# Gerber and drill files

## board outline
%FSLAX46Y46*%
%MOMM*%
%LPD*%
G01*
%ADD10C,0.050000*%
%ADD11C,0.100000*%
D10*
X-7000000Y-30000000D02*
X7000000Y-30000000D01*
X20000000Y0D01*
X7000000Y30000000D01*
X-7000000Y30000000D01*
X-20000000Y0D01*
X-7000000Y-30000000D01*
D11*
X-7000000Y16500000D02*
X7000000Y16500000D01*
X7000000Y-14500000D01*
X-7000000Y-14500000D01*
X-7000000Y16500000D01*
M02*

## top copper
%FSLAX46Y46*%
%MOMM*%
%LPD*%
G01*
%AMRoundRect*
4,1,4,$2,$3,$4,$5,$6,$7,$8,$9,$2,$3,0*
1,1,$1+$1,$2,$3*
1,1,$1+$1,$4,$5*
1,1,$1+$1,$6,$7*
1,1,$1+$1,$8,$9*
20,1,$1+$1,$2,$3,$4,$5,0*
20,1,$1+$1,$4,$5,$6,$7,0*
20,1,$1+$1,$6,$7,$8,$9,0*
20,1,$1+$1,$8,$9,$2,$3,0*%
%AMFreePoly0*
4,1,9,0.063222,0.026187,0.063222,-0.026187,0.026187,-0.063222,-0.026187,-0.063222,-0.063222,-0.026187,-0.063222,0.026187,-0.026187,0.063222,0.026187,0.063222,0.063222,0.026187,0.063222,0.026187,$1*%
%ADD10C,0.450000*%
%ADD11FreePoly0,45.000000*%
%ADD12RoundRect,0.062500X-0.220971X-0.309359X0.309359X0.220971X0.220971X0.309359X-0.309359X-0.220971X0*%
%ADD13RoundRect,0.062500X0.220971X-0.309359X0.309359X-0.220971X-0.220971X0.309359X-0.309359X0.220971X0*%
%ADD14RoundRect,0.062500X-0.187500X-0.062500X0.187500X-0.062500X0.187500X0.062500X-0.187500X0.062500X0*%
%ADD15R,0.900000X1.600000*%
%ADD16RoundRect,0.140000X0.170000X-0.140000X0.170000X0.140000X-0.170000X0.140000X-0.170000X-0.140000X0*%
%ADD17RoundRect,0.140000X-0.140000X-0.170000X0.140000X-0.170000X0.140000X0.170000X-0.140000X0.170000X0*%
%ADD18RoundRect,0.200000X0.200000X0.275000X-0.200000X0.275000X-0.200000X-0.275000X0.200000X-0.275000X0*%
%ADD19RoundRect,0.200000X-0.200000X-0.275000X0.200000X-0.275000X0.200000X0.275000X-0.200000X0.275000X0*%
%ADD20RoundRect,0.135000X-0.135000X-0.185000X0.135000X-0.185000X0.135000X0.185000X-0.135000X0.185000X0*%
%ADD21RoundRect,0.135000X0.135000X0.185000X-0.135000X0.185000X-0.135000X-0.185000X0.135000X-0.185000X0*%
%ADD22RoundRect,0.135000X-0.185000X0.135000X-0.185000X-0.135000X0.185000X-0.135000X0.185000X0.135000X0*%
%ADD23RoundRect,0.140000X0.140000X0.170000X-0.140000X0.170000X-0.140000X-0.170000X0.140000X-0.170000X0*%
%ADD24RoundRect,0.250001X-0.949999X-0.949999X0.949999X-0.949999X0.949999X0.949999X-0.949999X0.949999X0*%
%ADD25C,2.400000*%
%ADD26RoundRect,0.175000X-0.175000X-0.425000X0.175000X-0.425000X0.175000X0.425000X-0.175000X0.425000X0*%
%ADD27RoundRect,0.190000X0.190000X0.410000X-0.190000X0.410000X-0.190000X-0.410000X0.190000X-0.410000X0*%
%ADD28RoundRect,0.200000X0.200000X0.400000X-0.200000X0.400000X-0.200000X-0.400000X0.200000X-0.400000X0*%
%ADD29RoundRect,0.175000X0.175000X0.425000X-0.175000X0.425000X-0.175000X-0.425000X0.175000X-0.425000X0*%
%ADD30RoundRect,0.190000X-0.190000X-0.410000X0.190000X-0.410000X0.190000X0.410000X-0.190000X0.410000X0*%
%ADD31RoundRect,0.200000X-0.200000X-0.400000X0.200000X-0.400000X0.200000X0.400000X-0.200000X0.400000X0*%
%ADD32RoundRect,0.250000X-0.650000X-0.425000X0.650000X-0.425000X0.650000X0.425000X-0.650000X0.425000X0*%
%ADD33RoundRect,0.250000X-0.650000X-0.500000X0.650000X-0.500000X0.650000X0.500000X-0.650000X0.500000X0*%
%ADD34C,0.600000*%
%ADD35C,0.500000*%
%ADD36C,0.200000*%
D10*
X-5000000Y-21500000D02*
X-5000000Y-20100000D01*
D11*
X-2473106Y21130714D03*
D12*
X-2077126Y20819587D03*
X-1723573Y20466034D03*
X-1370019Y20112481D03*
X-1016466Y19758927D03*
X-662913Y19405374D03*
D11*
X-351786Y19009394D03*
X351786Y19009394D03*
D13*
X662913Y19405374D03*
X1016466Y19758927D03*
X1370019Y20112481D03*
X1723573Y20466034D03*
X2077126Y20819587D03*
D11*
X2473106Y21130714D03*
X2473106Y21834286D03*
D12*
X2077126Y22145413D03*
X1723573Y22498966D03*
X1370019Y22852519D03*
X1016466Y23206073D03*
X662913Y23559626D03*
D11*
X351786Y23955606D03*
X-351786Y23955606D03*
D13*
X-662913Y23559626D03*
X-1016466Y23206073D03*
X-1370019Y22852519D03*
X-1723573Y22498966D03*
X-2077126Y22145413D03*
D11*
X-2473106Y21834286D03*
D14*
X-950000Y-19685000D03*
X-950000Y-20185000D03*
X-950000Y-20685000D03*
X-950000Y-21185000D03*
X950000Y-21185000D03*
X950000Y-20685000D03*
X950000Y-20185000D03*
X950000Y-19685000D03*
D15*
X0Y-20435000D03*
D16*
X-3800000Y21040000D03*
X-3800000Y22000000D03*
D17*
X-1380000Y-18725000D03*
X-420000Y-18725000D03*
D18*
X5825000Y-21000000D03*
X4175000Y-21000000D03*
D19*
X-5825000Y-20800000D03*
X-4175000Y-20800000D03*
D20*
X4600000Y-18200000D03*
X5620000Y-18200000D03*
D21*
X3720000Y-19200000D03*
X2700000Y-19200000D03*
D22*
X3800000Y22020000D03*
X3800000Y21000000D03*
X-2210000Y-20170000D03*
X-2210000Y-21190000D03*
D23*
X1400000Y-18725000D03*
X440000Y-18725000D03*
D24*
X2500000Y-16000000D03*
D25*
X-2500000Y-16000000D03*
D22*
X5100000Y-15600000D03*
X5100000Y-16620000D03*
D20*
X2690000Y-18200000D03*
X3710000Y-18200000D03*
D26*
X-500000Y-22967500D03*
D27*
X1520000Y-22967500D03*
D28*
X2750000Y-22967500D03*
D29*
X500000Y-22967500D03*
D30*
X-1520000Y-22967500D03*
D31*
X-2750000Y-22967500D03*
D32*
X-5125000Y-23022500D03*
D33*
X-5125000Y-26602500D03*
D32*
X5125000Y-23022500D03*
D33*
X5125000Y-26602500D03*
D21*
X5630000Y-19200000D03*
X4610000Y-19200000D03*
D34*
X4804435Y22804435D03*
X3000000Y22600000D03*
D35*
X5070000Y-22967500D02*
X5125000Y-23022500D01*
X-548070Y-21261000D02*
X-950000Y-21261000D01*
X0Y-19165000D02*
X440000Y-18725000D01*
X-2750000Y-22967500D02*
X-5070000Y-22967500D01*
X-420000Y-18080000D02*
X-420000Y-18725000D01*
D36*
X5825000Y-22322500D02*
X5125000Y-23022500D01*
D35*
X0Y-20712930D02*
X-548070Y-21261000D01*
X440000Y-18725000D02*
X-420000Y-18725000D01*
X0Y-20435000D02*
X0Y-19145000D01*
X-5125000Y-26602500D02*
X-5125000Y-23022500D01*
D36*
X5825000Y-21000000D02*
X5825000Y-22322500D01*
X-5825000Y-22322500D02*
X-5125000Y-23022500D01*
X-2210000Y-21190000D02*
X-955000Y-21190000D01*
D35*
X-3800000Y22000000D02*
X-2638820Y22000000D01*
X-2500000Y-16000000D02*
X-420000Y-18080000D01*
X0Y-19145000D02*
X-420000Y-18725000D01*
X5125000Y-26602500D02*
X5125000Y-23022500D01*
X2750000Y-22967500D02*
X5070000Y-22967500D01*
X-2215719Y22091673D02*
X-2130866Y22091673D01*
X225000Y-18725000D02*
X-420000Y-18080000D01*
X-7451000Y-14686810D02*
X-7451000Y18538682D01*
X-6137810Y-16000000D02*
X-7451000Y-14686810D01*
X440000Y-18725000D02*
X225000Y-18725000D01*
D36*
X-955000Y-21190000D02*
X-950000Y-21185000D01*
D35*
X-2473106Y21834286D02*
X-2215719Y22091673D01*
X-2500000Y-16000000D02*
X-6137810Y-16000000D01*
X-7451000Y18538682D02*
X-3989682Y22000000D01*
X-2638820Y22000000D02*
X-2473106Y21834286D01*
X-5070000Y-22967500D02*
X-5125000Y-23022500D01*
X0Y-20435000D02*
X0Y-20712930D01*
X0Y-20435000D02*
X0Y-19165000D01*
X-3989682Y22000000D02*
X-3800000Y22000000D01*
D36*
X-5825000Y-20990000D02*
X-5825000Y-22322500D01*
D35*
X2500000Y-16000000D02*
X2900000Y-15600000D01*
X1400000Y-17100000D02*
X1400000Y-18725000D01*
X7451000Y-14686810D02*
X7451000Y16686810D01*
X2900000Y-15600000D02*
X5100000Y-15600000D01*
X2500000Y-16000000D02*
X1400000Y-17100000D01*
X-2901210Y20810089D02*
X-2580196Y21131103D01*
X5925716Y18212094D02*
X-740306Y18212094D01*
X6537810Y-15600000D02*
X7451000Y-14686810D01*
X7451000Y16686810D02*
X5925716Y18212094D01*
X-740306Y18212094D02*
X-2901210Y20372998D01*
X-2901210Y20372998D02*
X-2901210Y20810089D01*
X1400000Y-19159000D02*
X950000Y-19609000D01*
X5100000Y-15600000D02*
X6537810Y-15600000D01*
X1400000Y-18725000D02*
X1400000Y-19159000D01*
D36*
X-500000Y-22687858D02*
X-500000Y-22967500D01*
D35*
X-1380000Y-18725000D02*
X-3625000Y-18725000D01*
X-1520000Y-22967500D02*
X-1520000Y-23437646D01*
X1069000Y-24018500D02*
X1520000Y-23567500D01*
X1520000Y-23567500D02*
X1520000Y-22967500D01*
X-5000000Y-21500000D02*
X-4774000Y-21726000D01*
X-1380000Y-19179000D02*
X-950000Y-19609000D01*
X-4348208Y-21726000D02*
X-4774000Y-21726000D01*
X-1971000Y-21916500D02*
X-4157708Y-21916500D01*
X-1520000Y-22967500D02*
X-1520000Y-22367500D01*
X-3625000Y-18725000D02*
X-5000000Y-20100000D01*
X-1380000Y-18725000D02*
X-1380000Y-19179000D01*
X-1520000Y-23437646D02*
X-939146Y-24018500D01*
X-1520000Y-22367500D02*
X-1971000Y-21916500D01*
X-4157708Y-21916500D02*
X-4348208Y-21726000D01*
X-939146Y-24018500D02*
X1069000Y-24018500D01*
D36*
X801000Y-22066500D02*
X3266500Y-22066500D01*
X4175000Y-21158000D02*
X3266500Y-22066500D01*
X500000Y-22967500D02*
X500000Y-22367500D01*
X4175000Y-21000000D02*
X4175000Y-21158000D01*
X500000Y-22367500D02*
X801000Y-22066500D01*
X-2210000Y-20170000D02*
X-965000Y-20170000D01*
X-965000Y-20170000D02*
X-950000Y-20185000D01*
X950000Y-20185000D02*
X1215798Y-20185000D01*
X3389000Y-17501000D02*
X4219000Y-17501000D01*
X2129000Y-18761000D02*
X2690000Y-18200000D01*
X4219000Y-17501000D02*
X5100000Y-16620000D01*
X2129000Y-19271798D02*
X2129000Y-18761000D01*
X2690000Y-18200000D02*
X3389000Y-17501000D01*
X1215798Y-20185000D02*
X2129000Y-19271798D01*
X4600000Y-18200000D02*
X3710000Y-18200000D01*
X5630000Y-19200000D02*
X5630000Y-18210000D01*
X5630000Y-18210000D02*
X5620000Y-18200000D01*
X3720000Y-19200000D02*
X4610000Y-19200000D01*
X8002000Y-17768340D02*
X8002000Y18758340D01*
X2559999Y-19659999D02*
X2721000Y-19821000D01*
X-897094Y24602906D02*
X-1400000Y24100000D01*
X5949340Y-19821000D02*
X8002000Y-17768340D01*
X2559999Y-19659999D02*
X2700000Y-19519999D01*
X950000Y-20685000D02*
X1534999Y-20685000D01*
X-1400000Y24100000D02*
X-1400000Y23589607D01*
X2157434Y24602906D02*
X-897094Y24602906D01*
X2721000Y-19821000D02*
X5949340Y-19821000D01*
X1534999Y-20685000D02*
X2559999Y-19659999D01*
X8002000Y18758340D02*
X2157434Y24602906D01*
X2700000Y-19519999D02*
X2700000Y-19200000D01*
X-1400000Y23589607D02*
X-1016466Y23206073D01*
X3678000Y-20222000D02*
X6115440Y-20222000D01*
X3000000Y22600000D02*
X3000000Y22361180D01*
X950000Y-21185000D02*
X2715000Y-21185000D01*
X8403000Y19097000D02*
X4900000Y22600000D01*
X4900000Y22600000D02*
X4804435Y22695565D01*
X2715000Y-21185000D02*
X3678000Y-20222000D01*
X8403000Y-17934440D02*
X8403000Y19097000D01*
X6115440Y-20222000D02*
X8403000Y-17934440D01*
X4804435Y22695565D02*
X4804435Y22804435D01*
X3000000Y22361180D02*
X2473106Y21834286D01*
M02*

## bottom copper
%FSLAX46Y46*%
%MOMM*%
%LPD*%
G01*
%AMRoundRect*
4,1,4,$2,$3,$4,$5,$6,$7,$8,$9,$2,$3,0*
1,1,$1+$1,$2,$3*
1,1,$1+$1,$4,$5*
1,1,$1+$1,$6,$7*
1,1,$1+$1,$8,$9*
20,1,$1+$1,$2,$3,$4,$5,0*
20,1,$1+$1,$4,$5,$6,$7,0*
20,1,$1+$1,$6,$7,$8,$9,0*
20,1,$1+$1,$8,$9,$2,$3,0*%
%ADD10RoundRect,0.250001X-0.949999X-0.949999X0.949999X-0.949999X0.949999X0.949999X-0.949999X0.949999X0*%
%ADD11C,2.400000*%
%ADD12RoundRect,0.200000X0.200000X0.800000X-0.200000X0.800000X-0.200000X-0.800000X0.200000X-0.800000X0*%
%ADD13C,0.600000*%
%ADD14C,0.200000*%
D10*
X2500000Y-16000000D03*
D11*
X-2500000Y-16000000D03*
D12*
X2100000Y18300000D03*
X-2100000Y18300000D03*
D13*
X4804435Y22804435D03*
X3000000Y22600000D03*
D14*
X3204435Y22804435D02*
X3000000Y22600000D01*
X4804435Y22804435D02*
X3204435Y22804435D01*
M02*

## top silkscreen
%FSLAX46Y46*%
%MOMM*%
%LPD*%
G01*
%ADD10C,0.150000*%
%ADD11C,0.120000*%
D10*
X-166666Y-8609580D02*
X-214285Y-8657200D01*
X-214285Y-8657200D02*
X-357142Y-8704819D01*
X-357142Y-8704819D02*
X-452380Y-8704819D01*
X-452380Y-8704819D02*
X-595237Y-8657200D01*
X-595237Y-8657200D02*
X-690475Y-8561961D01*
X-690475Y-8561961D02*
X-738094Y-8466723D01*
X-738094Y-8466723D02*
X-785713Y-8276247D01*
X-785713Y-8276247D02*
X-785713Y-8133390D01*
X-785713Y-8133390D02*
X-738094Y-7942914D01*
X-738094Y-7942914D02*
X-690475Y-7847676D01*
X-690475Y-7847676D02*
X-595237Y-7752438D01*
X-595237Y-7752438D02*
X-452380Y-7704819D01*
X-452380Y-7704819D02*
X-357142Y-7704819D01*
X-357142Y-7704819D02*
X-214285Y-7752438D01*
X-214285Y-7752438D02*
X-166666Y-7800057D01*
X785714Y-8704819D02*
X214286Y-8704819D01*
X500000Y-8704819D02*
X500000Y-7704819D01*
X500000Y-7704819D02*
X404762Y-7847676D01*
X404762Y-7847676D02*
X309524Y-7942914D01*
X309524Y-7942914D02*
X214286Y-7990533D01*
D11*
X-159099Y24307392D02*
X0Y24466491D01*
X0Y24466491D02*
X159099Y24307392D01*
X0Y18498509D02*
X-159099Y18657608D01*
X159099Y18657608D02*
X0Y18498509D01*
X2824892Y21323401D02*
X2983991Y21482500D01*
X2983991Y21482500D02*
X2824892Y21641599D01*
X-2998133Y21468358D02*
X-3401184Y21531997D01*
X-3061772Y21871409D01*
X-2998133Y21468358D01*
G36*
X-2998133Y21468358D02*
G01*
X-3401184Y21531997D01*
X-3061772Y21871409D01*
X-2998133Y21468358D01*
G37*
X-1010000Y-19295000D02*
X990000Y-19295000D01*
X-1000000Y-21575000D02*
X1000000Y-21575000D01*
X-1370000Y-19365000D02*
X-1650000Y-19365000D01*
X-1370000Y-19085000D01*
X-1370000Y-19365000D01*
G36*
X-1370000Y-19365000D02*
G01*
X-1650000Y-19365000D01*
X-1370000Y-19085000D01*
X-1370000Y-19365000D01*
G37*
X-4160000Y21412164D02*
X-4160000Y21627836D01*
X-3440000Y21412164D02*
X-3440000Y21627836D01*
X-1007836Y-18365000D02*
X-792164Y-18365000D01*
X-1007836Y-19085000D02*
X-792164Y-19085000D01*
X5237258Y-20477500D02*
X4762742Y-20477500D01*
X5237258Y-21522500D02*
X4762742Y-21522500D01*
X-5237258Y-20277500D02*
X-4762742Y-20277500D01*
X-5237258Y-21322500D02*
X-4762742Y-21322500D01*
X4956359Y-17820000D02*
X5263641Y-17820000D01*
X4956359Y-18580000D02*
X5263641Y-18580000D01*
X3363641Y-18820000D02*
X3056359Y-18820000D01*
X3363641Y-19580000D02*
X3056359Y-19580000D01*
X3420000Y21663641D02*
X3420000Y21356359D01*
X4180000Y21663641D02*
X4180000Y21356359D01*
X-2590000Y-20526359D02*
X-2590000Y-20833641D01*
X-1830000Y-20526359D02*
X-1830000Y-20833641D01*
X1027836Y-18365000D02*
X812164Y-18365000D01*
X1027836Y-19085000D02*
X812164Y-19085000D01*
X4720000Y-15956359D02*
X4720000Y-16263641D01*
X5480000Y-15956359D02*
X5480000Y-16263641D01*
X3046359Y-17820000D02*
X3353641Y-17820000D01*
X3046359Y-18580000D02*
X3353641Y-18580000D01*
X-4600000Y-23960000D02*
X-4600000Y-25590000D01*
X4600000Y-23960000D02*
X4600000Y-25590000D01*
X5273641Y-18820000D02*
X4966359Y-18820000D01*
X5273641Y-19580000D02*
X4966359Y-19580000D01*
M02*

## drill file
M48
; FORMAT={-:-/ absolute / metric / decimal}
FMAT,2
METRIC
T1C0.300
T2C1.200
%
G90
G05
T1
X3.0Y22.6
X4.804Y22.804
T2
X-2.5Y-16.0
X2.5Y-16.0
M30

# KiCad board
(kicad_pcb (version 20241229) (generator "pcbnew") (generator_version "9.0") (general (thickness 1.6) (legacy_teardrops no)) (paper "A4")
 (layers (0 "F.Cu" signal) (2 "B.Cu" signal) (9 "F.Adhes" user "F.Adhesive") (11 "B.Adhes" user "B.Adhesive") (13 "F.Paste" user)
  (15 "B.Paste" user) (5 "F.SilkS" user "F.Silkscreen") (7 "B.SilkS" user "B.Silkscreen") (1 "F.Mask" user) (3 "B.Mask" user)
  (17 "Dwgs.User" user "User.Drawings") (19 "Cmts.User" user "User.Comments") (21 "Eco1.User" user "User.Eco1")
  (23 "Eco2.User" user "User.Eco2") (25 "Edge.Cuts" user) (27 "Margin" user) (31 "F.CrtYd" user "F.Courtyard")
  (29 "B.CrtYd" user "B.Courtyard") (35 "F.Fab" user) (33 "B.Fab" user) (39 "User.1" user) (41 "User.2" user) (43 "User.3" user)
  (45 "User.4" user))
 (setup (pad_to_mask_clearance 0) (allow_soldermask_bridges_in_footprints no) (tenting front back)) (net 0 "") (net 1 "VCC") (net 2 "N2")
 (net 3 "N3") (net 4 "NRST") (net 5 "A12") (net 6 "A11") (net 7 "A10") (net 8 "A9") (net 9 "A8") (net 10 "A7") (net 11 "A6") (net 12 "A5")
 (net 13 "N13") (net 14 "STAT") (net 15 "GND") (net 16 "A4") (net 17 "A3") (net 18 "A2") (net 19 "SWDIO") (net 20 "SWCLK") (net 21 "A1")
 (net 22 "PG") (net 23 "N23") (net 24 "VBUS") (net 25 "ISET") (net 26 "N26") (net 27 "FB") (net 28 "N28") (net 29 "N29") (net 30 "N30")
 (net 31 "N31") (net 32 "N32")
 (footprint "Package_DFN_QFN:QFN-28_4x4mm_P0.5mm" (layer "F.Cu") (at 0 -21.4825 45)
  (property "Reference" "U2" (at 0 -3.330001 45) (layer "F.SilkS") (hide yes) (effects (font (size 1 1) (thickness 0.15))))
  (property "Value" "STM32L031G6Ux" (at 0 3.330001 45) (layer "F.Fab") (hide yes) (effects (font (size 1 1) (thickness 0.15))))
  (fp_line (start 1.885 -2.11) (end 2.11 -2.11) (stroke (width 0.12) (type solid)) (layer "F.SilkS"))
  (fp_line (start 2.11 -2.11) (end 2.11 -1.885) (stroke (width 0.12) (type solid)) (layer "F.SilkS"))
  (fp_line (start -2.11 2.11) (end -2.11 1.885) (stroke (width 0.12) (type solid)) (layer "F.SilkS"))
  (fp_line (start -1.885 2.11) (end -2.11 2.11) (stroke (width 0.12) (type solid)) (layer "F.SilkS"))
  (fp_line (start 1.885 2.11) (end 2.11 2.11) (stroke (width 0.12) (type solid)) (layer "F.SilkS"))
  (fp_line (start 2.11 2.11) (end 2.11 1.885) (stroke (width 0.12) (type solid)) (layer "F.SilkS"))
  (fp_poly (pts (xy -2.13 -2.11) (xy -2.370001 -2.44) (xy -1.89 -2.44)) (stroke (width 0.12) (type solid)) (fill yes) (layer "F.SilkS"))
  (pad "1" smd custom (at -1.9975 -1.5 45) (size 0.136863 0.136863) (layers "F.Cu" "F.Mask" "F.Paste") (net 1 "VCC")
   (options (clearance outline) (anchor circle)) (primitives))
  (pad "2" smd roundrect (at -1.9375 -1 45) (size 0.875 0.25) (layers "F.Cu" "F.Mask" "F.Paste") (roundrect_rratio 0.25) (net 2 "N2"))
  (pad "3" smd roundrect (at -1.9375 -0.5 45) (size 0.875 0.25) (layers "F.Cu" "F.Mask" "F.Paste") (roundrect_rratio 0.25) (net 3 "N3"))
  (pad "4" smd roundrect (at -1.937499 0 45) (size 0.875 0.25) (layers "F.Cu" "F.Mask" "F.Paste") (roundrect_rratio 0.25) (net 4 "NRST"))
  (pad "5" smd roundrect (at -1.9375 0.5 45) (size 0.875 0.25) (layers "F.Cu" "F.Mask" "F.Paste") (roundrect_rratio 0.25) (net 1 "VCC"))
  (pad "6" smd roundrect (at -1.9375 1 45) (size 0.875 0.25) (layers "F.Cu" "F.Mask" "F.Paste") (roundrect_rratio 0.25) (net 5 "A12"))
  (pad "7" smd custom (at -1.9975 1.5 45) (size 0.136863 0.136863) (layers "F.Cu" "F.Mask" "F.Paste") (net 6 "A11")
   (options (clearance outline) (anchor circle)) (primitives))
  (pad "8" smd custom (at -1.5 1.9975 45) (size 0.136863 0.136863) (layers "F.Cu" "F.Mask" "F.Paste") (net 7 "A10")
   (options (clearance outline) (anchor circle)) (primitives))
  (pad "9" smd roundrect (at -1 1.9375 45) (size 0.25 0.875) (layers "F.Cu" "F.Mask" "F.Paste") (roundrect_rratio 0.25) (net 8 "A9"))
  (pad "10" smd roundrect (at -0.5 1.9375 45) (size 0.25 0.875) (layers "F.Cu" "F.Mask" "F.Paste") (roundrect_rratio 0.25) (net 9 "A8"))
  (pad "11" smd roundrect (at 0 1.937499 45) (size 0.25 0.875) (layers "F.Cu" "F.Mask" "F.Paste") (roundrect_rratio 0.25) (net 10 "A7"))
  (pad "12" smd roundrect (at 0.5 1.9375 45) (size 0.25 0.875) (layers "F.Cu" "F.Mask" "F.Paste") (roundrect_rratio 0.25) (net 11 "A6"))
  (pad "13" smd roundrect (at 1 1.9375 45) (size 0.25 0.875) (layers "F.Cu" "F.Mask" "F.Paste") (roundrect_rratio 0.25) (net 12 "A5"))
  (pad "14" smd custom (at 1.5 1.9975 45) (size 0.136863 0.136863) (layers "F.Cu" "F.Mask" "F.Paste") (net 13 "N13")
   (options (clearance outline) (anchor circle)) (primitives))
  (pad "15" smd custom (at 1.9975 1.5 45) (size 0.136863 0.136863) (layers "F.Cu" "F.Mask" "F.Paste") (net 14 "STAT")
   (options (clearance outline) (anchor circle)) (primitives))
  (pad "16" smd roundrect (at 1.9375 1 45) (size 0.875 0.25) (layers "F.Cu" "F.Mask" "F.Paste") (roundrect_rratio 0.25) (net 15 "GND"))
  (pad "17" smd roundrect (at 1.9375 0.5 45) (size 0.875 0.25) (layers "F.Cu" "F.Mask" "F.Paste") (roundrect_rratio 0.25) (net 1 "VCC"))
  (pad "18" smd roundrect (at 1.937499 0 45) (size 0.875 0.25) (layers "F.Cu" "F.Mask" "F.Paste") (roundrect_rratio 0.25) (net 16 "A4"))
  (pad "19" smd roundrect (at 1.9375 -0.5 45) (size 0.875 0.25) (layers "F.Cu" "F.Mask" "F.Paste") (roundrect_rratio 0.25) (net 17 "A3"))
  (pad "20" smd roundrect (at 1.9375 -1 45) (size 0.875 0.25) (layers "F.Cu" "F.Mask" "F.Paste") (roundrect_rratio 0.25) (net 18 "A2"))
  (pad "21" smd custom (at 1.9975 -1.5 45) (size 0.136863 0.136863) (layers "F.Cu" "F.Mask" "F.Paste") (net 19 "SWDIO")
   (options (clearance outline) (anchor circle)) (primitives))
  (pad "22" smd custom (at 1.5 -1.9975 45) (size 0.136863 0.136863) (layers "F.Cu" "F.Mask" "F.Paste") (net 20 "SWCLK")
   (options (clearance outline) (anchor circle)) (primitives))
  (pad "23" smd roundrect (at 1 -1.9375 45) (size 0.25 0.875) (layers "F.Cu" "F.Mask" "F.Paste") (roundrect_rratio 0.25) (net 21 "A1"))
  (pad "24" smd roundrect (at 0.5 -1.9375 45) (size 0.25 0.875) (layers "F.Cu" "F.Mask" "F.Paste") (roundrect_rratio 0.25) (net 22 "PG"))
  (pad "25" smd roundrect (at 0 -1.937499 45) (size 0.25 0.875) (layers "F.Cu" "F.Mask" "F.Paste") (roundrect_rratio 0.25) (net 4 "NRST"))
  (pad "26" smd roundrect (at -0.5 -1.9375 45) (size 0.25 0.875) (layers "F.Cu" "F.Mask" "F.Paste") (roundrect_rratio 0.25) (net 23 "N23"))
  (pad "27" smd roundrect (at -1 -1.9375 45) (size 0.25 0.875) (layers "F.Cu" "F.Mask" "F.Paste") (roundrect_rratio 0.25) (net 15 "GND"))
  (pad "28" smd custom (at -1.5 -1.9975 45) (size 0.136863 0.136863) (layers "F.Cu" "F.Mask" "F.Paste") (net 15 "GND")
   (options (clearance outline) (anchor circle)) (primitives)))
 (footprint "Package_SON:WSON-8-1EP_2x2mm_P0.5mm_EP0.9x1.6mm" (layer "F.Cu") (at 0 20.435)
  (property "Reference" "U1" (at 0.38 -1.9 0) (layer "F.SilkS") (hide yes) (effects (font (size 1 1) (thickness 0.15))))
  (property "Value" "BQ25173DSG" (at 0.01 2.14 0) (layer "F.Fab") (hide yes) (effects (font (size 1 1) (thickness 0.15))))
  (fp_line (start -1.01 -1.14) (end 0.99 -1.14) (stroke (width 0.12) (type solid)) (layer "F.SilkS"))
  (fp_line (start -1 1.14) (end 1 1.14) (stroke (width 0.12) (type solid)) (layer "F.SilkS"))
  (fp_poly
   (pts (xy -1.37 -1.07) (xy -1.65 -1.07) (xy -1.37 -1.35) (xy -1.37 -1.07)) (stroke (width 0.12) (type solid)) (fill yes) (layer "F.SilkS"))
  (pad "" smd rect (at 0 -0.4) (size 0.75 0.65) (layers "F.Paste"))
  (pad "" smd rect (at 0 0.4) (size 0.75 0.65) (layers "F.Paste"))
  (pad "1" smd roundrect (at -0.95 -0.75) (size 0.5 0.25) (layers "F.Cu" "F.Mask" "F.Paste") (roundrect_rratio 0.25) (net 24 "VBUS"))
  (pad "2" smd roundrect (at -0.95 -0.25) (size 0.5 0.25) (layers "F.Cu" "F.Mask" "F.Paste") (roundrect_rratio 0.25) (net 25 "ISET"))
  (pad "3" smd roundrect (at -0.95 0.25) (size 0.5 0.25) (layers "F.Cu" "F.Mask" "F.Paste") (roundrect_rratio 0.25) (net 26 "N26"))
  (pad "4" smd roundrect (at -0.95 0.75) (size 0.5 0.25) (layers "F.Cu" "F.Mask" "F.Paste") (roundrect_rratio 0.25) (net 15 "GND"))
  (pad "5" smd roundrect (at 0.95 0.75) (size 0.5 0.25) (layers "F.Cu" "F.Mask" "F.Paste") (roundrect_rratio 0.25) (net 14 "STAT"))
  (pad "6" smd roundrect (at 0.95 0.25) (size 0.5 0.25) (layers "F.Cu" "F.Mask" "F.Paste") (roundrect_rratio 0.25) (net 22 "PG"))
  (pad "7" smd roundrect (at 0.95 -0.25) (size 0.5 0.25) (layers "F.Cu" "F.Mask" "F.Paste") (roundrect_rratio 0.25) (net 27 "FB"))
  (pad "8" smd roundrect (at 0.95 -0.75) (size 0.5 0.25) (layers "F.Cu" "F.Mask" "F.Paste") (roundrect_rratio 0.25) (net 1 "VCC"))
  (pad "9" smd rect (at 0 0) (size 0.9 1.6) (layers "F.Cu" "F.Mask") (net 15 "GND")))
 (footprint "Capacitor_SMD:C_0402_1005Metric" (layer "F.Cu") (at -3.8 -21.52 90)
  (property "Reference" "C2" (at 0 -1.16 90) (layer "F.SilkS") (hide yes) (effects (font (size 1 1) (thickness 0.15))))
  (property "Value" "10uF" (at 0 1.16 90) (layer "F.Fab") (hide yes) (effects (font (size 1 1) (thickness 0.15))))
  (fp_line (start -0.107836 -0.36) (end 0.107836 -0.36) (stroke (width 0.12) (type solid)) (layer "F.SilkS"))
  (fp_line (start -0.107836 0.36) (end 0.107836 0.36) (stroke (width 0.12) (type solid)) (layer "F.SilkS"))
  (pad "1" smd roundrect (at -0.48 0 90) (size 0.56 0.62) (layers "F.Cu" "F.Mask" "F.Paste") (roundrect_rratio 0.25) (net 1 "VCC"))
  (pad "2" smd roundrect (at 0.48 0 90) (size 0.56 0.62) (layers "F.Cu" "F.Mask" "F.Paste") (roundrect_rratio 0.25) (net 15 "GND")))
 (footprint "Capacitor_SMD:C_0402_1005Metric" (layer "F.Cu") (at -0.9 18.725)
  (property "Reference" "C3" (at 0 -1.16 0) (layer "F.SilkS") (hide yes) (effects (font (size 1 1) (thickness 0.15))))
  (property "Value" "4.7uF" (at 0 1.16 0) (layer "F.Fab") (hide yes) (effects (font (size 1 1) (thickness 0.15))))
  (fp_line (start -0.107836 -0.36) (end 0.107836 -0.36) (stroke (width 0.12) (type solid)) (layer "F.SilkS"))
  (fp_line (start -0.107836 0.36) (end 0.107836 0.36) (stroke (width 0.12) (type solid)) (layer "F.SilkS"))
  (pad "1" smd roundrect (at -0.48 0) (size 0.56 0.62) (layers "F.Cu" "F.Mask" "F.Paste") (roundrect_rratio 0.25) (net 24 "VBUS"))
  (pad "2" smd roundrect (at 0.48 0) (size 0.56 0.62) (layers "F.Cu" "F.Mask" "F.Paste") (roundrect_rratio 0.25) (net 15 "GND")))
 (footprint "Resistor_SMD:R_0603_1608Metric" (layer "F.Cu") (at 5 21 180)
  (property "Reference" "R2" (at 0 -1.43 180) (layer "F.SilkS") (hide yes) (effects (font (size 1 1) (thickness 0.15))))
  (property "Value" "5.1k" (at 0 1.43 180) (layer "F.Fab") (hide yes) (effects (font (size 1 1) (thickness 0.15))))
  (fp_line (start -0.237258 0.5225) (end 0.237258 0.5225) (stroke (width 0.12) (type solid)) (layer "F.SilkS"))
  (fp_line (start -0.237258 -0.5225) (end 0.237258 -0.5225) (stroke (width 0.12) (type solid)) (layer "F.SilkS"))
  (pad "1" smd roundrect (at -0.825 0 180) (size 0.8 0.95) (layers "F.Cu" "F.Mask" "F.Paste") (roundrect_rratio 0.25) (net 15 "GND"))
  (pad "2" smd roundrect (at 0.825 0 180) (size 0.8 0.95) (layers "F.Cu" "F.Mask" "F.Paste") (roundrect_rratio 0.25) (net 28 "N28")))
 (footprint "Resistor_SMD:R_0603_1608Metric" (layer "F.Cu") (at -5 20.8)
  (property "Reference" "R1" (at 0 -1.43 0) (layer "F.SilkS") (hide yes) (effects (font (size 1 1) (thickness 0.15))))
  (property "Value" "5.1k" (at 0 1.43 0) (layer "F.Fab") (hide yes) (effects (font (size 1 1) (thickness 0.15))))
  (fp_line (start -0.237258 -0.5225) (end 0.237258 -0.5225) (stroke (width 0.12) (type solid)) (layer "F.SilkS"))
  (fp_line (start -0.237258 0.5225) (end 0.237258 0.5225) (stroke (width 0.12) (type solid)) (layer "F.SilkS"))
  (pad "1" smd roundrect (at -0.825 0) (size 0.8 0.95) (layers "F.Cu" "F.Mask" "F.Paste") (roundrect_rratio 0.25) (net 15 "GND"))
  (pad "2" smd roundrect (at 0.825 0) (size 0.8 0.95) (layers "F.Cu" "F.Mask" "F.Paste") (roundrect_rratio 0.25) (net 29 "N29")))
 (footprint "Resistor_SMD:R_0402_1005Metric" (layer "F.Cu") (at 5.11 18.2)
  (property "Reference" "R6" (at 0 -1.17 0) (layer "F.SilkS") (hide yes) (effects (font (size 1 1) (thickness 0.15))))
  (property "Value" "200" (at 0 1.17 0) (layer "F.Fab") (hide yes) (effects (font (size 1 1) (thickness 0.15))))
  (fp_line (start -0.153641 -0.38) (end 0.153641 -0.38) (stroke (width 0.12) (type solid)) (layer "F.SilkS"))
  (fp_line (start -0.153641 0.38) (end 0.153641 0.38) (stroke (width 0.12) (type solid)) (layer "F.SilkS"))
  (pad "1" smd roundrect (at -0.51 0) (size 0.54 0.64) (layers "F.Cu" "F.Mask" "F.Paste") (roundrect_rratio 0.25) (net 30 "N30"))
  (pad "2" smd roundrect (at 0.51 0) (size 0.54 0.64) (layers "F.Cu" "F.Mask" "F.Paste") (roundrect_rratio 0.25) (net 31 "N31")))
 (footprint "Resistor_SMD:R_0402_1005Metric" (layer "F.Cu") (at 3.21 19.2 180)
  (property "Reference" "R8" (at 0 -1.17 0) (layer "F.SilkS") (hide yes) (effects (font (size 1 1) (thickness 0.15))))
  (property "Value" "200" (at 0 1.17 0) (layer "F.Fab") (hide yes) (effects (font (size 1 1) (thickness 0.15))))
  (fp_line (start -0.153641 0.38) (end 0.153641 0.38) (stroke (width 0.12) (type solid)) (layer "F.SilkS"))
  (fp_line (start -0.153641 -0.38) (end 0.153641 -0.38) (stroke (width 0.12) (type solid)) (layer "F.SilkS"))
  (pad "1" smd roundrect (at -0.51 0 180) (size 0.54 0.64) (layers "F.Cu" "F.Mask" "F.Paste") (roundrect_rratio 0.25) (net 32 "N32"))
  (pad "2" smd roundrect (at 0.51 0 180) (size 0.54 0.64) (layers "F.Cu" "F.Mask" "F.Paste") (roundrect_rratio 0.25) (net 22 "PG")))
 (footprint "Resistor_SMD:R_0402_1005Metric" (layer "F.Cu") (at 3.8 -21.51 -90)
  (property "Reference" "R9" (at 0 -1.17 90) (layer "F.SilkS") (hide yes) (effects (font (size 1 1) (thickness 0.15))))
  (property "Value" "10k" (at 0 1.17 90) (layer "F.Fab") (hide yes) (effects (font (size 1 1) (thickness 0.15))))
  (fp_line (start -0.153641 0.38) (end 0.153641 0.38) (stroke (width 0.12) (type solid)) (layer "F.SilkS"))
  (fp_line (start -0.153641 -0.38) (end 0.153641 -0.38) (stroke (width 0.12) (type solid)) (layer "F.SilkS"))
  (pad "1" smd roundrect (at -0.51 0 270) (size 0.54 0.64) (layers "F.Cu" "F.Mask" "F.Paste") (roundrect_rratio 0.25) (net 14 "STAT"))
  (pad "2" smd roundrect (at 0.51 0 270) (size 0.54 0.64) (layers "F.Cu" "F.Mask" "F.Paste") (roundrect_rratio 0.25) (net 1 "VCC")))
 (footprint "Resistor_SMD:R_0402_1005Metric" (layer "F.Cu") (at -2.21 20.68 -90)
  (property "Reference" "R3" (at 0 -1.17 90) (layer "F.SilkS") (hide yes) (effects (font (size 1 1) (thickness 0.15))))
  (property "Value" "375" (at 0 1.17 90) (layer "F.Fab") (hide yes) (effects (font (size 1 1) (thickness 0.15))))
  (fp_line (start -0.153641 0.38) (end 0.153641 0.38) (stroke (width 0.12) (type solid)) (layer "F.SilkS"))
  (fp_line (start -0.153641 -0.38) (end 0.153641 -0.38) (stroke (width 0.12) (type solid)) (layer "F.SilkS"))
  (pad "1" smd roundrect (at -0.51 0 270) (size 0.54 0.64) (layers "F.Cu" "F.Mask" "F.Paste") (roundrect_rratio 0.25) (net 25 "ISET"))
  (pad "2" smd roundrect (at 0.51 0 270) (size 0.54 0.64) (layers "F.Cu" "F.Mask" "F.Paste") (roundrect_rratio 0.25) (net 15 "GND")))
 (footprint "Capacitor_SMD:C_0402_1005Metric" (layer "F.Cu") (at 0.92 18.725 180)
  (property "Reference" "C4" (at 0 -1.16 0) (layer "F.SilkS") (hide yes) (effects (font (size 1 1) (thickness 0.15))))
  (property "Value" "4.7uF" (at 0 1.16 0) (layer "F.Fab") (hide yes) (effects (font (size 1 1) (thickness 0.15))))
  (fp_line (start -0.107836 0.36) (end 0.107836 0.36) (stroke (width 0.12) (type solid)) (layer "F.SilkS"))
  (fp_line (start -0.107836 -0.36) (end 0.107836 -0.36) (stroke (width 0.12) (type solid)) (layer "F.SilkS"))
  (pad "1" smd roundrect (at -0.48 0 180) (size 0.56 0.62) (layers "F.Cu" "F.Mask" "F.Paste") (roundrect_rratio 0.25) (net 1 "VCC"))
  (pad "2" smd roundrect (at 0.48 0 180) (size 0.56 0.62) (layers "F.Cu" "F.Mask" "F.Paste") (roundrect_rratio 0.25) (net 15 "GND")))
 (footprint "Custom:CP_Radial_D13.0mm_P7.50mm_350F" (layer "F.Cu") (at 0 16)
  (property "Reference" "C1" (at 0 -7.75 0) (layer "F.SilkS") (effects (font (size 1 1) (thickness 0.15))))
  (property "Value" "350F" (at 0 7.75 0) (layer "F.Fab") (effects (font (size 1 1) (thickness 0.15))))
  (fp_rect (start -7 -32.5) (end 7 -1.5) (stroke (width 0.1) (type default)) (fill no) (layer "Edge.Cuts"))
  (pad "1" thru_hole roundrect (at 2.5 0) (size 2.4 2.4) (drill 1.2) (layers "*.Cu" "*.Mask") (remove_unused_layers no)
   (roundrect_rratio 0.104167) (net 1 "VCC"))
  (pad "2" thru_hole circle (at -2.5 0) (size 2.4 2.4) (drill 1.2) (layers "*.Cu" "*.Mask") (remove_unused_layers no) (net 15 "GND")))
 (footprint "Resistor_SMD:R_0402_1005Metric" (layer "F.Cu") (at 5.1 16.11 -90)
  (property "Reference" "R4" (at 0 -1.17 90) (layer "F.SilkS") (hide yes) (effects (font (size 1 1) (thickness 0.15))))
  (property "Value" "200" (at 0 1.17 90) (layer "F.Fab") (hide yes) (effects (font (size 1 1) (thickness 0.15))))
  (fp_line (start -0.153641 0.38) (end 0.153641 0.38) (stroke (width 0.12) (type solid)) (layer "F.SilkS"))
  (fp_line (start -0.153641 -0.38) (end 0.153641 -0.38) (stroke (width 0.12) (type solid)) (layer "F.SilkS"))
  (pad "1" smd roundrect (at -0.51 0 270) (size 0.54 0.64) (layers "F.Cu" "F.Mask" "F.Paste") (roundrect_rratio 0.25) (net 1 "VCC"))
  (pad "2" smd roundrect (at 0.51 0 270) (size 0.54 0.64) (layers "F.Cu" "F.Mask" "F.Paste") (roundrect_rratio 0.25) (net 27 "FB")))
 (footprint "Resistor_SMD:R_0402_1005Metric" (layer "F.Cu") (at 3.2 18.2)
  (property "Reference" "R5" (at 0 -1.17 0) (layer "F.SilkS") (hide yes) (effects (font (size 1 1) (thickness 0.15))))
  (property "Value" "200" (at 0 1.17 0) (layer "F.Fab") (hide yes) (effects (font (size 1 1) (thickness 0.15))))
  (fp_line (start -0.153641 -0.38) (end 0.153641 -0.38) (stroke (width 0.12) (type solid)) (layer "F.SilkS"))
  (fp_line (start -0.153641 0.38) (end 0.153641 0.38) (stroke (width 0.12) (type solid)) (layer "F.SilkS"))
  (pad "1" smd roundrect (at -0.51 0) (size 0.54 0.64) (layers "F.Cu" "F.Mask" "F.Paste") (roundrect_rratio 0.25) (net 27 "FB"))
  (pad "2" smd roundrect (at 0.51 0) (size 0.54 0.64) (layers "F.Cu" "F.Mask" "F.Paste") (roundrect_rratio 0.25) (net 30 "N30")))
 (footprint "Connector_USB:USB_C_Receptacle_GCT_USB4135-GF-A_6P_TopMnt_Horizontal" (layer "F.Cu") (at 0 26)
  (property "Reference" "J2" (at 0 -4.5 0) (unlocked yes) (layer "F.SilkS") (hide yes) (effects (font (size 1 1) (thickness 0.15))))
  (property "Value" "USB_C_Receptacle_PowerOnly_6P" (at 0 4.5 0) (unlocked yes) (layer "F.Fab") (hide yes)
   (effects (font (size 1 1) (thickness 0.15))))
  (fp_line (start -4.6 -2.04) (end -4.6 -0.41) (stroke (width 0.12) (type solid)) (layer "F.SilkS"))
  (fp_line (start 4.6 -2.04) (end 4.6 -0.41) (stroke (width 0.12) (type solid)) (layer "F.SilkS"))
  (pad "A5" smd roundrect (at -0.5 -3.0325) (size 0.7 1.2) (layers "F.Cu" "F.Mask" "F.Paste") (roundrect_rratio 0.25) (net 29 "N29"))
  (pad "A9" smd roundrect (at 1.52 -3.0325 180) (size 0.76 1.2) (layers "F.Cu" "F.Mask" "F.Paste") (roundrect_rratio 0.25) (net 24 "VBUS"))
  (pad "A12" smd roundrect (at 2.75 -3.0325 180) (size 0.8 1.2) (layers "F.Cu" "F.Mask" "F.Paste") (roundrect_rratio 0.25) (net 15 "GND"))
  (pad "B5" smd roundrect (at 0.5 -3.0325 180) (size 0.7 1.2) (layers "F.Cu" "F.Mask" "F.Paste") (roundrect_rratio 0.25) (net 28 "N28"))
  (pad "B9" smd roundrect (at -1.52 -3.0325) (size 0.76 1.2) (layers "F.Cu" "F.Mask" "F.Paste") (roundrect_rratio 0.25) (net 24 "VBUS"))
  (pad "B12" smd roundrect (at -2.75 -3.0325) (size 0.8 1.2) (layers "F.Cu" "F.Mask" "F.Paste") (roundrect_rratio 0.25) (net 15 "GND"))
  (pad "S1" smd roundrect (at -5.125 -2.9775) (size 1.8 1.35) (layers "F.Cu" "F.Mask" "F.Paste") (roundrect_rratio 0.1851851852)
   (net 15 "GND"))
  (pad "S1" smd roundrect (at -5.125 0.6025) (size 1.8 1.5) (layers "F.Cu" "F.Mask" "F.Paste") (roundrect_rratio 0.1666666667)
   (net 15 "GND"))
  (pad "S1" smd roundrect (at 5.125 -2.9775) (size 1.8 1.35) (layers "F.Cu" "F.Mask" "F.Paste") (roundrect_rratio 0.1851851852)
   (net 15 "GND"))
  (pad "S1" smd roundrect (at 5.125 0.6025) (size 1.8 1.5) (layers "F.Cu" "F.Mask" "F.Paste") (roundrect_rratio 0.1666666667) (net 15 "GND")))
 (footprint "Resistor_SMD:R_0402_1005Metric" (layer "F.Cu") (at 5.12 19.2 180)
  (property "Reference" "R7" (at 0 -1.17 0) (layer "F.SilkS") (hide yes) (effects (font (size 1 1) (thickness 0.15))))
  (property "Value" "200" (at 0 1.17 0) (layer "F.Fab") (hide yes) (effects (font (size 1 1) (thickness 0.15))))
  (fp_line (start -0.153641 0.38) (end 0.153641 0.38) (stroke (width 0.12) (type solid)) (layer "F.SilkS"))
  (fp_line (start -0.153641 -0.38) (end 0.153641 -0.38) (stroke (width 0.12) (type solid)) (layer "F.SilkS"))
  (pad "1" smd roundrect (at -0.51 0 180) (size 0.54 0.64) (layers "F.Cu" "F.Mask" "F.Paste") (roundrect_rratio 0.25) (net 31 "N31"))
  (pad "2" smd roundrect (at 0.51 0 180) (size 0.54 0.64) (layers "F.Cu" "F.Mask" "F.Paste") (roundrect_rratio 0.25) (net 32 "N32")))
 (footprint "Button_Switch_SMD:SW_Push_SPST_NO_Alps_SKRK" (layer "B.Cu") (at 0 -18.3 180)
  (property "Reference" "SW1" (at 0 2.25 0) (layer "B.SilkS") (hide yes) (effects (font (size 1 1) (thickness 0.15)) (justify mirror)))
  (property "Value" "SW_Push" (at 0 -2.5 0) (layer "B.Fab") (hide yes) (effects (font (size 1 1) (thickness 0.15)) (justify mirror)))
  (pad "1" smd roundrect (at -2.1 0 180) (size 0.8 2) (layers "B.Cu" "B.Mask" "B.Paste") (roundrect_rratio 0.25) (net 15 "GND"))
  (pad "2" smd roundrect (at 2.1 0 180) (size 0.8 2) (layers "B.Cu" "B.Mask" "B.Paste") (roundrect_rratio 0.25) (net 23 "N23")))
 (gr_line (start -5 21.5) (end -5 20.1) (stroke (width 0.45) (type default)) (layer "F.Cu") (net 24))
 (gr_poly
  (pts (xy -7 30) (xy 7 30) (xy 20 0) (xy 7 -30) (xy -7 -30) (xy -20 0)) (stroke (width 0.05) (type solid)) (fill no) (layer "Edge.Cuts"))
 (segment (start 5.07 22.9675) (end 5.125 23.0225) (width 0.5) (layer "F.Cu") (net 15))
 (segment (start -0.54807 21.261) (end -0.95 21.261) (width 0.5) (layer "F.Cu") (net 15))
 (segment (start 0 19.165) (end 0.44 18.725) (width 0.5) (layer "F.Cu") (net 15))
 (segment (start -2.75 22.9675) (end -5.07 22.9675) (width 0.5) (layer "F.Cu") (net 15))
 (segment (start -0.42 18.08) (end -0.42 18.725) (width 0.5) (layer "F.Cu") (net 15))
 (segment (start 5.825 22.3225) (end 5.125 23.0225) (width 0.2) (layer "F.Cu") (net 15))
 (segment (start 0 20.71293) (end -0.54807 21.261) (width 0.5) (layer "F.Cu") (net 15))
 (segment (start 0.44 18.725) (end -0.42 18.725) (width 0.5) (layer "F.Cu") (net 15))
 (segment (start 0 20.435) (end 0 19.145) (width 0.5) (layer "F.Cu") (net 15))
 (segment (start -5.125 26.6025) (end -5.125 23.0225) (width 0.5) (layer "F.Cu") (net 15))
 (segment (start 5.825 21) (end 5.825 22.3225) (width 0.2) (layer "F.Cu") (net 15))
 (segment (start -5.825 22.3225) (end -5.125 23.0225) (width 0.2) (layer "F.Cu") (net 15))
 (segment (start -2.21 21.19) (end -0.955 21.19) (width 0.2) (layer "F.Cu") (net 15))
 (segment (start -3.8 -22) (end -2.63882 -22) (width 0.5) (layer "F.Cu") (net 15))
 (segment (start -2.5 16) (end -0.42 18.08) (width 0.5) (layer "F.Cu") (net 15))
 (segment (start 0 19.145) (end -0.42 18.725) (width 0.5) (layer "F.Cu") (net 15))
 (segment (start 5.125 26.6025) (end 5.125 23.0225) (width 0.5) (layer "F.Cu") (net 15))
 (segment (start 2.75 22.9675) (end 5.07 22.9675) (width 0.5) (layer "F.Cu") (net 15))
 (segment (start -2.215719 -22.091673) (end -2.130866 -22.091673) (width 0.5) (layer "F.Cu") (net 15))
 (segment (start 0.225 18.725) (end -0.42 18.08) (width 0.5) (layer "F.Cu") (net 15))
 (segment (start -7.451 14.68681) (end -7.451 -18.538682) (width 0.5) (layer "F.Cu") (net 15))
 (segment (start -6.13781 16) (end -7.451 14.68681) (width 0.5) (layer "F.Cu") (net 15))
 (segment (start 0.44 18.725) (end 0.225 18.725) (width 0.5) (layer "F.Cu") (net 15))
 (segment (start -0.955 21.19) (end -0.95 21.185) (width 0.2) (layer "F.Cu") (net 15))
 (segment (start -2.473106 -21.834286) (end -2.215719 -22.091673) (width 0.5) (layer "F.Cu") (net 15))
 (segment (start -2.5 16) (end -6.13781 16) (width 0.5) (layer "F.Cu") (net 15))
 (segment (start -7.451 -18.538682) (end -3.989682 -22) (width 0.5) (layer "F.Cu") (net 15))
 (segment (start -2.63882 -22) (end -2.473106 -21.834286) (width 0.5) (layer "F.Cu") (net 15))
 (segment (start -5.07 22.9675) (end -5.125 23.0225) (width 0.5) (layer "F.Cu") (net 15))
 (segment (start 0 20.435) (end 0 20.71293) (width 0.5) (layer "F.Cu") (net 15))
 (segment (start 0 20.435) (end 0 19.165) (width 0.5) (layer "F.Cu") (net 15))
 (segment (start -3.989682 -22) (end -3.8 -22) (width 0.5) (layer "F.Cu") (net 15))
 (segment (start -5.825 20.99) (end -5.825 22.3225) (width 0.2) (layer "F.Cu") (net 15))
 (segment (start 2.5 16) (end 2.9 15.6) (width 0.5) (layer "F.Cu") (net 1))
 (segment (start 1.4 17.1) (end 1.4 18.725) (width 0.5) (layer "F.Cu") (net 1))
 (segment (start 7.451 14.68681) (end 7.451 -16.68681) (width 0.5) (layer "F.Cu") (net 1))
 (segment (start 2.9 15.6) (end 5.1 15.6) (width 0.5) (layer "F.Cu") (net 1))
 (segment (start 2.5 16) (end 1.4 17.1) (width 0.5) (layer "F.Cu") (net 1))
 (segment (start -2.90121 -20.810089) (end -2.580196 -21.131103) (width 0.5) (layer "F.Cu") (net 1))
 (segment (start 5.925716 -18.212094) (end -0.740306 -18.212094) (width 0.5) (layer "F.Cu") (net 1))
 (segment (start 6.53781 15.6) (end 7.451 14.68681) (width 0.5) (layer "F.Cu") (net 1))
 (segment (start 7.451 -16.68681) (end 5.925716 -18.212094) (width 0.5) (layer "F.Cu") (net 1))
 (segment (start -0.740306 -18.212094) (end -2.90121 -20.372998) (width 0.5) (layer "F.Cu") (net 1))
 (segment (start -2.90121 -20.372998) (end -2.90121 -20.810089) (width 0.5) (layer "F.Cu") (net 1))
 (segment (start 1.4 19.159) (end 0.95 19.609) (width 0.5) (layer "F.Cu") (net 1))
 (segment (start 5.1 15.6) (end 6.53781 15.6) (width 0.5) (layer "F.Cu") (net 1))
 (segment (start 1.4 18.725) (end 1.4 19.159) (width 0.5) (layer "F.Cu") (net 1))
 (segment (start -0.5 22.687858) (end -0.5 22.9675) (width 0.2) (layer "F.Cu") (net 29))
 (segment (start -1.38 18.725) (end -3.625 18.725) (width 0.5) (layer "F.Cu") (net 24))
 (segment (start -1.52 22.9675) (end -1.52 23.437646) (width 0.5) (layer "F.Cu") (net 24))
 (segment (start 1.069 24.0185) (end 1.52 23.5675) (width 0.5) (layer "F.Cu") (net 24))
 (segment (start 1.52 23.5675) (end 1.52 22.9675) (width 0.5) (layer "F.Cu") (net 24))
 (segment (start -5 21.5) (end -4.774 21.726) (width 0.5) (layer "F.Cu") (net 24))
 (segment (start -1.38 19.179) (end -0.95 19.609) (width 0.5) (layer "F.Cu") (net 24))
 (segment (start -4.348208 21.726) (end -4.774 21.726) (width 0.5) (layer "F.Cu") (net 24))
 (segment (start -1.971 21.9165) (end -4.157708 21.9165) (width 0.5) (layer "F.Cu") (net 24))
 (segment (start -1.52 22.9675) (end -1.52 22.3675) (width 0.5) (layer "F.Cu") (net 24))
 (segment (start -3.625 18.725) (end -5 20.1) (width 0.5) (layer "F.Cu") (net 24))
 (segment (start -1.38 18.725) (end -1.38 19.179) (width 0.5) (layer "F.Cu") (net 24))
 (segment (start -1.52 23.437646) (end -0.939146 24.0185) (width 0.5) (layer "F.Cu") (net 24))
 (segment (start -1.52 22.3675) (end -1.971 21.9165) (width 0.5) (layer "F.Cu") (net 24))
 (segment (start -4.157708 21.9165) (end -4.348208 21.726) (width 0.5) (layer "F.Cu") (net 24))
 (segment (start -0.939146 24.0185) (end 1.069 24.0185) (width 0.5) (layer "F.Cu") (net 24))
 (segment (start 0.801 22.0665) (end 3.2665 22.0665) (width 0.2) (layer "F.Cu") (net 28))
 (segment (start 4.175 21.158) (end 3.2665 22.0665) (width 0.2) (layer "F.Cu") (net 28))
 (segment (start 0.5 22.9675) (end 0.5 22.3675) (width 0.2) (layer "F.Cu") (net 28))
 (segment (start 4.175 21) (end 4.175 21.158) (width 0.2) (layer "F.Cu") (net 28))
 (segment (start 0.5 22.3675) (end 0.801 22.0665) (width 0.2) (layer "F.Cu") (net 28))
 (segment (start -2.21 20.17) (end -0.965 20.17) (width 0.2) (layer "F.Cu") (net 25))
 (segment (start -0.965 20.17) (end -0.95 20.185) (width 0.2) (layer "F.Cu") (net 25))
 (segment (start 0.95 20.185) (end 1.215798 20.185) (width 0.2) (layer "F.Cu") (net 27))
 (segment (start 3.389 17.501) (end 4.219 17.501) (width 0.2) (layer "F.Cu") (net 27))
 (segment (start 2.129 18.761) (end 2.69 18.2) (width 0.2) (layer "F.Cu") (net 27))
 (segment (start 4.219 17.501) (end 5.1 16.62) (width 0.2) (layer "F.Cu") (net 27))
 (segment (start 2.129 19.271798) (end 2.129 18.761) (width 0.2) (layer "F.Cu") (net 27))
 (segment (start 2.69 18.2) (end 3.389 17.501) (width 0.2) (layer "F.Cu") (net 27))
 (segment (start 1.215798 20.185) (end 2.129 19.271798) (width 0.2) (layer "F.Cu") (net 27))
 (segment (start 4.6 18.2) (end 3.71 18.2) (width 0.2) (layer "F.Cu") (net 30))
 (segment (start 5.63 19.2) (end 5.63 18.21) (width 0.2) (layer "F.Cu") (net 31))
 (segment (start 5.63 18.21) (end 5.62 18.2) (width 0.2) (layer "F.Cu") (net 31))
 (segment (start 3.72 19.2) (end 4.61 19.2) (width 0.2) (layer "F.Cu") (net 32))
 (segment (start 8.002 17.76834) (end 8.002 -18.75834) (width 0.2) (layer "F.Cu") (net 22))
 (segment (start 2.559999 19.659999) (end 2.721 19.821) (width 0.2) (layer "F.Cu") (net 22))
 (segment (start -0.897094 -24.602906) (end -1.4 -24.1) (width 0.2) (layer "F.Cu") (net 22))
 (segment (start 5.94934 19.821) (end 8.002 17.76834) (width 0.2) (layer "F.Cu") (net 22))
 (segment (start 2.559999 19.659999) (end 2.7 19.519999) (width 0.2) (layer "F.Cu") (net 22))
 (segment (start 0.95 20.685) (end 1.534999 20.685) (width 0.2) (layer "F.Cu") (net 22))
 (segment (start -1.4 -24.1) (end -1.4 -23.589607) (width 0.2) (layer "F.Cu") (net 22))
 (segment (start 2.157434 -24.602906) (end -0.897094 -24.602906) (width 0.2) (layer "F.Cu") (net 22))
 (segment (start 2.721 19.821) (end 5.94934 19.821) (width 0.2) (layer "F.Cu") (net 22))
 (segment (start 1.534999 20.685) (end 2.559999 19.659999) (width 0.2) (layer "F.Cu") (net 22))
 (segment (start 8.002 -18.75834) (end 2.157434 -24.602906) (width 0.2) (layer "F.Cu") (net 22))
 (segment (start 2.7 19.519999) (end 2.7 19.2) (width 0.2) (layer "F.Cu") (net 22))
 (segment (start -1.4 -23.589607) (end -1.016466 -23.206073) (width 0.2) (layer "F.Cu") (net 22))
 (segment (start 3.678 20.222) (end 6.11544 20.222) (width 0.2) (layer "F.Cu") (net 14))
 (segment (start 3 -22.6) (end 3 -22.36118) (width 0.2) (layer "F.Cu") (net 14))
 (segment (start 0.95 21.185) (end 2.715 21.185) (width 0.2) (layer "F.Cu") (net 14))
 (segment (start 8.403 -19.097) (end 4.9 -22.6) (width 0.2) (layer "F.Cu") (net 14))
 (segment (start 4.9 -22.6) (end 4.804435 -22.695565) (width 0.2) (layer "F.Cu") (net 14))
 (segment (start 2.715 21.185) (end 3.678 20.222) (width 0.2) (layer "F.Cu") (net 14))
 (segment (start 8.403 17.93444) (end 8.403 -19.097) (width 0.2) (layer "F.Cu") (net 14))
 (segment (start 6.11544 20.222) (end 8.403 17.93444) (width 0.2) (layer "F.Cu") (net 14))
 (segment (start 4.804435 -22.695565) (end 4.804435 -22.804435) (width 0.2) (layer "F.Cu") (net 14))
 (segment (start 3 -22.36118) (end 2.473106 -21.834286) (width 0.2) (layer "F.Cu") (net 14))
 (via (at 4.804435 -22.804435) (size 0.6) (drill 0.3) (layers "F.Cu" "B.Cu") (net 14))
 (via (at 3 -22.6) (size 0.6) (drill 0.3) (layers "F.Cu" "B.Cu") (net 14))
 (segment (start 3.204435 -22.804435) (end 3 -22.6) (width 0.2) (layer "B.Cu") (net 14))
 (segment (start 4.804435 -22.804435) (end 3.204435 -22.804435) (width 0.2) (layer "B.Cu") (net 14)))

